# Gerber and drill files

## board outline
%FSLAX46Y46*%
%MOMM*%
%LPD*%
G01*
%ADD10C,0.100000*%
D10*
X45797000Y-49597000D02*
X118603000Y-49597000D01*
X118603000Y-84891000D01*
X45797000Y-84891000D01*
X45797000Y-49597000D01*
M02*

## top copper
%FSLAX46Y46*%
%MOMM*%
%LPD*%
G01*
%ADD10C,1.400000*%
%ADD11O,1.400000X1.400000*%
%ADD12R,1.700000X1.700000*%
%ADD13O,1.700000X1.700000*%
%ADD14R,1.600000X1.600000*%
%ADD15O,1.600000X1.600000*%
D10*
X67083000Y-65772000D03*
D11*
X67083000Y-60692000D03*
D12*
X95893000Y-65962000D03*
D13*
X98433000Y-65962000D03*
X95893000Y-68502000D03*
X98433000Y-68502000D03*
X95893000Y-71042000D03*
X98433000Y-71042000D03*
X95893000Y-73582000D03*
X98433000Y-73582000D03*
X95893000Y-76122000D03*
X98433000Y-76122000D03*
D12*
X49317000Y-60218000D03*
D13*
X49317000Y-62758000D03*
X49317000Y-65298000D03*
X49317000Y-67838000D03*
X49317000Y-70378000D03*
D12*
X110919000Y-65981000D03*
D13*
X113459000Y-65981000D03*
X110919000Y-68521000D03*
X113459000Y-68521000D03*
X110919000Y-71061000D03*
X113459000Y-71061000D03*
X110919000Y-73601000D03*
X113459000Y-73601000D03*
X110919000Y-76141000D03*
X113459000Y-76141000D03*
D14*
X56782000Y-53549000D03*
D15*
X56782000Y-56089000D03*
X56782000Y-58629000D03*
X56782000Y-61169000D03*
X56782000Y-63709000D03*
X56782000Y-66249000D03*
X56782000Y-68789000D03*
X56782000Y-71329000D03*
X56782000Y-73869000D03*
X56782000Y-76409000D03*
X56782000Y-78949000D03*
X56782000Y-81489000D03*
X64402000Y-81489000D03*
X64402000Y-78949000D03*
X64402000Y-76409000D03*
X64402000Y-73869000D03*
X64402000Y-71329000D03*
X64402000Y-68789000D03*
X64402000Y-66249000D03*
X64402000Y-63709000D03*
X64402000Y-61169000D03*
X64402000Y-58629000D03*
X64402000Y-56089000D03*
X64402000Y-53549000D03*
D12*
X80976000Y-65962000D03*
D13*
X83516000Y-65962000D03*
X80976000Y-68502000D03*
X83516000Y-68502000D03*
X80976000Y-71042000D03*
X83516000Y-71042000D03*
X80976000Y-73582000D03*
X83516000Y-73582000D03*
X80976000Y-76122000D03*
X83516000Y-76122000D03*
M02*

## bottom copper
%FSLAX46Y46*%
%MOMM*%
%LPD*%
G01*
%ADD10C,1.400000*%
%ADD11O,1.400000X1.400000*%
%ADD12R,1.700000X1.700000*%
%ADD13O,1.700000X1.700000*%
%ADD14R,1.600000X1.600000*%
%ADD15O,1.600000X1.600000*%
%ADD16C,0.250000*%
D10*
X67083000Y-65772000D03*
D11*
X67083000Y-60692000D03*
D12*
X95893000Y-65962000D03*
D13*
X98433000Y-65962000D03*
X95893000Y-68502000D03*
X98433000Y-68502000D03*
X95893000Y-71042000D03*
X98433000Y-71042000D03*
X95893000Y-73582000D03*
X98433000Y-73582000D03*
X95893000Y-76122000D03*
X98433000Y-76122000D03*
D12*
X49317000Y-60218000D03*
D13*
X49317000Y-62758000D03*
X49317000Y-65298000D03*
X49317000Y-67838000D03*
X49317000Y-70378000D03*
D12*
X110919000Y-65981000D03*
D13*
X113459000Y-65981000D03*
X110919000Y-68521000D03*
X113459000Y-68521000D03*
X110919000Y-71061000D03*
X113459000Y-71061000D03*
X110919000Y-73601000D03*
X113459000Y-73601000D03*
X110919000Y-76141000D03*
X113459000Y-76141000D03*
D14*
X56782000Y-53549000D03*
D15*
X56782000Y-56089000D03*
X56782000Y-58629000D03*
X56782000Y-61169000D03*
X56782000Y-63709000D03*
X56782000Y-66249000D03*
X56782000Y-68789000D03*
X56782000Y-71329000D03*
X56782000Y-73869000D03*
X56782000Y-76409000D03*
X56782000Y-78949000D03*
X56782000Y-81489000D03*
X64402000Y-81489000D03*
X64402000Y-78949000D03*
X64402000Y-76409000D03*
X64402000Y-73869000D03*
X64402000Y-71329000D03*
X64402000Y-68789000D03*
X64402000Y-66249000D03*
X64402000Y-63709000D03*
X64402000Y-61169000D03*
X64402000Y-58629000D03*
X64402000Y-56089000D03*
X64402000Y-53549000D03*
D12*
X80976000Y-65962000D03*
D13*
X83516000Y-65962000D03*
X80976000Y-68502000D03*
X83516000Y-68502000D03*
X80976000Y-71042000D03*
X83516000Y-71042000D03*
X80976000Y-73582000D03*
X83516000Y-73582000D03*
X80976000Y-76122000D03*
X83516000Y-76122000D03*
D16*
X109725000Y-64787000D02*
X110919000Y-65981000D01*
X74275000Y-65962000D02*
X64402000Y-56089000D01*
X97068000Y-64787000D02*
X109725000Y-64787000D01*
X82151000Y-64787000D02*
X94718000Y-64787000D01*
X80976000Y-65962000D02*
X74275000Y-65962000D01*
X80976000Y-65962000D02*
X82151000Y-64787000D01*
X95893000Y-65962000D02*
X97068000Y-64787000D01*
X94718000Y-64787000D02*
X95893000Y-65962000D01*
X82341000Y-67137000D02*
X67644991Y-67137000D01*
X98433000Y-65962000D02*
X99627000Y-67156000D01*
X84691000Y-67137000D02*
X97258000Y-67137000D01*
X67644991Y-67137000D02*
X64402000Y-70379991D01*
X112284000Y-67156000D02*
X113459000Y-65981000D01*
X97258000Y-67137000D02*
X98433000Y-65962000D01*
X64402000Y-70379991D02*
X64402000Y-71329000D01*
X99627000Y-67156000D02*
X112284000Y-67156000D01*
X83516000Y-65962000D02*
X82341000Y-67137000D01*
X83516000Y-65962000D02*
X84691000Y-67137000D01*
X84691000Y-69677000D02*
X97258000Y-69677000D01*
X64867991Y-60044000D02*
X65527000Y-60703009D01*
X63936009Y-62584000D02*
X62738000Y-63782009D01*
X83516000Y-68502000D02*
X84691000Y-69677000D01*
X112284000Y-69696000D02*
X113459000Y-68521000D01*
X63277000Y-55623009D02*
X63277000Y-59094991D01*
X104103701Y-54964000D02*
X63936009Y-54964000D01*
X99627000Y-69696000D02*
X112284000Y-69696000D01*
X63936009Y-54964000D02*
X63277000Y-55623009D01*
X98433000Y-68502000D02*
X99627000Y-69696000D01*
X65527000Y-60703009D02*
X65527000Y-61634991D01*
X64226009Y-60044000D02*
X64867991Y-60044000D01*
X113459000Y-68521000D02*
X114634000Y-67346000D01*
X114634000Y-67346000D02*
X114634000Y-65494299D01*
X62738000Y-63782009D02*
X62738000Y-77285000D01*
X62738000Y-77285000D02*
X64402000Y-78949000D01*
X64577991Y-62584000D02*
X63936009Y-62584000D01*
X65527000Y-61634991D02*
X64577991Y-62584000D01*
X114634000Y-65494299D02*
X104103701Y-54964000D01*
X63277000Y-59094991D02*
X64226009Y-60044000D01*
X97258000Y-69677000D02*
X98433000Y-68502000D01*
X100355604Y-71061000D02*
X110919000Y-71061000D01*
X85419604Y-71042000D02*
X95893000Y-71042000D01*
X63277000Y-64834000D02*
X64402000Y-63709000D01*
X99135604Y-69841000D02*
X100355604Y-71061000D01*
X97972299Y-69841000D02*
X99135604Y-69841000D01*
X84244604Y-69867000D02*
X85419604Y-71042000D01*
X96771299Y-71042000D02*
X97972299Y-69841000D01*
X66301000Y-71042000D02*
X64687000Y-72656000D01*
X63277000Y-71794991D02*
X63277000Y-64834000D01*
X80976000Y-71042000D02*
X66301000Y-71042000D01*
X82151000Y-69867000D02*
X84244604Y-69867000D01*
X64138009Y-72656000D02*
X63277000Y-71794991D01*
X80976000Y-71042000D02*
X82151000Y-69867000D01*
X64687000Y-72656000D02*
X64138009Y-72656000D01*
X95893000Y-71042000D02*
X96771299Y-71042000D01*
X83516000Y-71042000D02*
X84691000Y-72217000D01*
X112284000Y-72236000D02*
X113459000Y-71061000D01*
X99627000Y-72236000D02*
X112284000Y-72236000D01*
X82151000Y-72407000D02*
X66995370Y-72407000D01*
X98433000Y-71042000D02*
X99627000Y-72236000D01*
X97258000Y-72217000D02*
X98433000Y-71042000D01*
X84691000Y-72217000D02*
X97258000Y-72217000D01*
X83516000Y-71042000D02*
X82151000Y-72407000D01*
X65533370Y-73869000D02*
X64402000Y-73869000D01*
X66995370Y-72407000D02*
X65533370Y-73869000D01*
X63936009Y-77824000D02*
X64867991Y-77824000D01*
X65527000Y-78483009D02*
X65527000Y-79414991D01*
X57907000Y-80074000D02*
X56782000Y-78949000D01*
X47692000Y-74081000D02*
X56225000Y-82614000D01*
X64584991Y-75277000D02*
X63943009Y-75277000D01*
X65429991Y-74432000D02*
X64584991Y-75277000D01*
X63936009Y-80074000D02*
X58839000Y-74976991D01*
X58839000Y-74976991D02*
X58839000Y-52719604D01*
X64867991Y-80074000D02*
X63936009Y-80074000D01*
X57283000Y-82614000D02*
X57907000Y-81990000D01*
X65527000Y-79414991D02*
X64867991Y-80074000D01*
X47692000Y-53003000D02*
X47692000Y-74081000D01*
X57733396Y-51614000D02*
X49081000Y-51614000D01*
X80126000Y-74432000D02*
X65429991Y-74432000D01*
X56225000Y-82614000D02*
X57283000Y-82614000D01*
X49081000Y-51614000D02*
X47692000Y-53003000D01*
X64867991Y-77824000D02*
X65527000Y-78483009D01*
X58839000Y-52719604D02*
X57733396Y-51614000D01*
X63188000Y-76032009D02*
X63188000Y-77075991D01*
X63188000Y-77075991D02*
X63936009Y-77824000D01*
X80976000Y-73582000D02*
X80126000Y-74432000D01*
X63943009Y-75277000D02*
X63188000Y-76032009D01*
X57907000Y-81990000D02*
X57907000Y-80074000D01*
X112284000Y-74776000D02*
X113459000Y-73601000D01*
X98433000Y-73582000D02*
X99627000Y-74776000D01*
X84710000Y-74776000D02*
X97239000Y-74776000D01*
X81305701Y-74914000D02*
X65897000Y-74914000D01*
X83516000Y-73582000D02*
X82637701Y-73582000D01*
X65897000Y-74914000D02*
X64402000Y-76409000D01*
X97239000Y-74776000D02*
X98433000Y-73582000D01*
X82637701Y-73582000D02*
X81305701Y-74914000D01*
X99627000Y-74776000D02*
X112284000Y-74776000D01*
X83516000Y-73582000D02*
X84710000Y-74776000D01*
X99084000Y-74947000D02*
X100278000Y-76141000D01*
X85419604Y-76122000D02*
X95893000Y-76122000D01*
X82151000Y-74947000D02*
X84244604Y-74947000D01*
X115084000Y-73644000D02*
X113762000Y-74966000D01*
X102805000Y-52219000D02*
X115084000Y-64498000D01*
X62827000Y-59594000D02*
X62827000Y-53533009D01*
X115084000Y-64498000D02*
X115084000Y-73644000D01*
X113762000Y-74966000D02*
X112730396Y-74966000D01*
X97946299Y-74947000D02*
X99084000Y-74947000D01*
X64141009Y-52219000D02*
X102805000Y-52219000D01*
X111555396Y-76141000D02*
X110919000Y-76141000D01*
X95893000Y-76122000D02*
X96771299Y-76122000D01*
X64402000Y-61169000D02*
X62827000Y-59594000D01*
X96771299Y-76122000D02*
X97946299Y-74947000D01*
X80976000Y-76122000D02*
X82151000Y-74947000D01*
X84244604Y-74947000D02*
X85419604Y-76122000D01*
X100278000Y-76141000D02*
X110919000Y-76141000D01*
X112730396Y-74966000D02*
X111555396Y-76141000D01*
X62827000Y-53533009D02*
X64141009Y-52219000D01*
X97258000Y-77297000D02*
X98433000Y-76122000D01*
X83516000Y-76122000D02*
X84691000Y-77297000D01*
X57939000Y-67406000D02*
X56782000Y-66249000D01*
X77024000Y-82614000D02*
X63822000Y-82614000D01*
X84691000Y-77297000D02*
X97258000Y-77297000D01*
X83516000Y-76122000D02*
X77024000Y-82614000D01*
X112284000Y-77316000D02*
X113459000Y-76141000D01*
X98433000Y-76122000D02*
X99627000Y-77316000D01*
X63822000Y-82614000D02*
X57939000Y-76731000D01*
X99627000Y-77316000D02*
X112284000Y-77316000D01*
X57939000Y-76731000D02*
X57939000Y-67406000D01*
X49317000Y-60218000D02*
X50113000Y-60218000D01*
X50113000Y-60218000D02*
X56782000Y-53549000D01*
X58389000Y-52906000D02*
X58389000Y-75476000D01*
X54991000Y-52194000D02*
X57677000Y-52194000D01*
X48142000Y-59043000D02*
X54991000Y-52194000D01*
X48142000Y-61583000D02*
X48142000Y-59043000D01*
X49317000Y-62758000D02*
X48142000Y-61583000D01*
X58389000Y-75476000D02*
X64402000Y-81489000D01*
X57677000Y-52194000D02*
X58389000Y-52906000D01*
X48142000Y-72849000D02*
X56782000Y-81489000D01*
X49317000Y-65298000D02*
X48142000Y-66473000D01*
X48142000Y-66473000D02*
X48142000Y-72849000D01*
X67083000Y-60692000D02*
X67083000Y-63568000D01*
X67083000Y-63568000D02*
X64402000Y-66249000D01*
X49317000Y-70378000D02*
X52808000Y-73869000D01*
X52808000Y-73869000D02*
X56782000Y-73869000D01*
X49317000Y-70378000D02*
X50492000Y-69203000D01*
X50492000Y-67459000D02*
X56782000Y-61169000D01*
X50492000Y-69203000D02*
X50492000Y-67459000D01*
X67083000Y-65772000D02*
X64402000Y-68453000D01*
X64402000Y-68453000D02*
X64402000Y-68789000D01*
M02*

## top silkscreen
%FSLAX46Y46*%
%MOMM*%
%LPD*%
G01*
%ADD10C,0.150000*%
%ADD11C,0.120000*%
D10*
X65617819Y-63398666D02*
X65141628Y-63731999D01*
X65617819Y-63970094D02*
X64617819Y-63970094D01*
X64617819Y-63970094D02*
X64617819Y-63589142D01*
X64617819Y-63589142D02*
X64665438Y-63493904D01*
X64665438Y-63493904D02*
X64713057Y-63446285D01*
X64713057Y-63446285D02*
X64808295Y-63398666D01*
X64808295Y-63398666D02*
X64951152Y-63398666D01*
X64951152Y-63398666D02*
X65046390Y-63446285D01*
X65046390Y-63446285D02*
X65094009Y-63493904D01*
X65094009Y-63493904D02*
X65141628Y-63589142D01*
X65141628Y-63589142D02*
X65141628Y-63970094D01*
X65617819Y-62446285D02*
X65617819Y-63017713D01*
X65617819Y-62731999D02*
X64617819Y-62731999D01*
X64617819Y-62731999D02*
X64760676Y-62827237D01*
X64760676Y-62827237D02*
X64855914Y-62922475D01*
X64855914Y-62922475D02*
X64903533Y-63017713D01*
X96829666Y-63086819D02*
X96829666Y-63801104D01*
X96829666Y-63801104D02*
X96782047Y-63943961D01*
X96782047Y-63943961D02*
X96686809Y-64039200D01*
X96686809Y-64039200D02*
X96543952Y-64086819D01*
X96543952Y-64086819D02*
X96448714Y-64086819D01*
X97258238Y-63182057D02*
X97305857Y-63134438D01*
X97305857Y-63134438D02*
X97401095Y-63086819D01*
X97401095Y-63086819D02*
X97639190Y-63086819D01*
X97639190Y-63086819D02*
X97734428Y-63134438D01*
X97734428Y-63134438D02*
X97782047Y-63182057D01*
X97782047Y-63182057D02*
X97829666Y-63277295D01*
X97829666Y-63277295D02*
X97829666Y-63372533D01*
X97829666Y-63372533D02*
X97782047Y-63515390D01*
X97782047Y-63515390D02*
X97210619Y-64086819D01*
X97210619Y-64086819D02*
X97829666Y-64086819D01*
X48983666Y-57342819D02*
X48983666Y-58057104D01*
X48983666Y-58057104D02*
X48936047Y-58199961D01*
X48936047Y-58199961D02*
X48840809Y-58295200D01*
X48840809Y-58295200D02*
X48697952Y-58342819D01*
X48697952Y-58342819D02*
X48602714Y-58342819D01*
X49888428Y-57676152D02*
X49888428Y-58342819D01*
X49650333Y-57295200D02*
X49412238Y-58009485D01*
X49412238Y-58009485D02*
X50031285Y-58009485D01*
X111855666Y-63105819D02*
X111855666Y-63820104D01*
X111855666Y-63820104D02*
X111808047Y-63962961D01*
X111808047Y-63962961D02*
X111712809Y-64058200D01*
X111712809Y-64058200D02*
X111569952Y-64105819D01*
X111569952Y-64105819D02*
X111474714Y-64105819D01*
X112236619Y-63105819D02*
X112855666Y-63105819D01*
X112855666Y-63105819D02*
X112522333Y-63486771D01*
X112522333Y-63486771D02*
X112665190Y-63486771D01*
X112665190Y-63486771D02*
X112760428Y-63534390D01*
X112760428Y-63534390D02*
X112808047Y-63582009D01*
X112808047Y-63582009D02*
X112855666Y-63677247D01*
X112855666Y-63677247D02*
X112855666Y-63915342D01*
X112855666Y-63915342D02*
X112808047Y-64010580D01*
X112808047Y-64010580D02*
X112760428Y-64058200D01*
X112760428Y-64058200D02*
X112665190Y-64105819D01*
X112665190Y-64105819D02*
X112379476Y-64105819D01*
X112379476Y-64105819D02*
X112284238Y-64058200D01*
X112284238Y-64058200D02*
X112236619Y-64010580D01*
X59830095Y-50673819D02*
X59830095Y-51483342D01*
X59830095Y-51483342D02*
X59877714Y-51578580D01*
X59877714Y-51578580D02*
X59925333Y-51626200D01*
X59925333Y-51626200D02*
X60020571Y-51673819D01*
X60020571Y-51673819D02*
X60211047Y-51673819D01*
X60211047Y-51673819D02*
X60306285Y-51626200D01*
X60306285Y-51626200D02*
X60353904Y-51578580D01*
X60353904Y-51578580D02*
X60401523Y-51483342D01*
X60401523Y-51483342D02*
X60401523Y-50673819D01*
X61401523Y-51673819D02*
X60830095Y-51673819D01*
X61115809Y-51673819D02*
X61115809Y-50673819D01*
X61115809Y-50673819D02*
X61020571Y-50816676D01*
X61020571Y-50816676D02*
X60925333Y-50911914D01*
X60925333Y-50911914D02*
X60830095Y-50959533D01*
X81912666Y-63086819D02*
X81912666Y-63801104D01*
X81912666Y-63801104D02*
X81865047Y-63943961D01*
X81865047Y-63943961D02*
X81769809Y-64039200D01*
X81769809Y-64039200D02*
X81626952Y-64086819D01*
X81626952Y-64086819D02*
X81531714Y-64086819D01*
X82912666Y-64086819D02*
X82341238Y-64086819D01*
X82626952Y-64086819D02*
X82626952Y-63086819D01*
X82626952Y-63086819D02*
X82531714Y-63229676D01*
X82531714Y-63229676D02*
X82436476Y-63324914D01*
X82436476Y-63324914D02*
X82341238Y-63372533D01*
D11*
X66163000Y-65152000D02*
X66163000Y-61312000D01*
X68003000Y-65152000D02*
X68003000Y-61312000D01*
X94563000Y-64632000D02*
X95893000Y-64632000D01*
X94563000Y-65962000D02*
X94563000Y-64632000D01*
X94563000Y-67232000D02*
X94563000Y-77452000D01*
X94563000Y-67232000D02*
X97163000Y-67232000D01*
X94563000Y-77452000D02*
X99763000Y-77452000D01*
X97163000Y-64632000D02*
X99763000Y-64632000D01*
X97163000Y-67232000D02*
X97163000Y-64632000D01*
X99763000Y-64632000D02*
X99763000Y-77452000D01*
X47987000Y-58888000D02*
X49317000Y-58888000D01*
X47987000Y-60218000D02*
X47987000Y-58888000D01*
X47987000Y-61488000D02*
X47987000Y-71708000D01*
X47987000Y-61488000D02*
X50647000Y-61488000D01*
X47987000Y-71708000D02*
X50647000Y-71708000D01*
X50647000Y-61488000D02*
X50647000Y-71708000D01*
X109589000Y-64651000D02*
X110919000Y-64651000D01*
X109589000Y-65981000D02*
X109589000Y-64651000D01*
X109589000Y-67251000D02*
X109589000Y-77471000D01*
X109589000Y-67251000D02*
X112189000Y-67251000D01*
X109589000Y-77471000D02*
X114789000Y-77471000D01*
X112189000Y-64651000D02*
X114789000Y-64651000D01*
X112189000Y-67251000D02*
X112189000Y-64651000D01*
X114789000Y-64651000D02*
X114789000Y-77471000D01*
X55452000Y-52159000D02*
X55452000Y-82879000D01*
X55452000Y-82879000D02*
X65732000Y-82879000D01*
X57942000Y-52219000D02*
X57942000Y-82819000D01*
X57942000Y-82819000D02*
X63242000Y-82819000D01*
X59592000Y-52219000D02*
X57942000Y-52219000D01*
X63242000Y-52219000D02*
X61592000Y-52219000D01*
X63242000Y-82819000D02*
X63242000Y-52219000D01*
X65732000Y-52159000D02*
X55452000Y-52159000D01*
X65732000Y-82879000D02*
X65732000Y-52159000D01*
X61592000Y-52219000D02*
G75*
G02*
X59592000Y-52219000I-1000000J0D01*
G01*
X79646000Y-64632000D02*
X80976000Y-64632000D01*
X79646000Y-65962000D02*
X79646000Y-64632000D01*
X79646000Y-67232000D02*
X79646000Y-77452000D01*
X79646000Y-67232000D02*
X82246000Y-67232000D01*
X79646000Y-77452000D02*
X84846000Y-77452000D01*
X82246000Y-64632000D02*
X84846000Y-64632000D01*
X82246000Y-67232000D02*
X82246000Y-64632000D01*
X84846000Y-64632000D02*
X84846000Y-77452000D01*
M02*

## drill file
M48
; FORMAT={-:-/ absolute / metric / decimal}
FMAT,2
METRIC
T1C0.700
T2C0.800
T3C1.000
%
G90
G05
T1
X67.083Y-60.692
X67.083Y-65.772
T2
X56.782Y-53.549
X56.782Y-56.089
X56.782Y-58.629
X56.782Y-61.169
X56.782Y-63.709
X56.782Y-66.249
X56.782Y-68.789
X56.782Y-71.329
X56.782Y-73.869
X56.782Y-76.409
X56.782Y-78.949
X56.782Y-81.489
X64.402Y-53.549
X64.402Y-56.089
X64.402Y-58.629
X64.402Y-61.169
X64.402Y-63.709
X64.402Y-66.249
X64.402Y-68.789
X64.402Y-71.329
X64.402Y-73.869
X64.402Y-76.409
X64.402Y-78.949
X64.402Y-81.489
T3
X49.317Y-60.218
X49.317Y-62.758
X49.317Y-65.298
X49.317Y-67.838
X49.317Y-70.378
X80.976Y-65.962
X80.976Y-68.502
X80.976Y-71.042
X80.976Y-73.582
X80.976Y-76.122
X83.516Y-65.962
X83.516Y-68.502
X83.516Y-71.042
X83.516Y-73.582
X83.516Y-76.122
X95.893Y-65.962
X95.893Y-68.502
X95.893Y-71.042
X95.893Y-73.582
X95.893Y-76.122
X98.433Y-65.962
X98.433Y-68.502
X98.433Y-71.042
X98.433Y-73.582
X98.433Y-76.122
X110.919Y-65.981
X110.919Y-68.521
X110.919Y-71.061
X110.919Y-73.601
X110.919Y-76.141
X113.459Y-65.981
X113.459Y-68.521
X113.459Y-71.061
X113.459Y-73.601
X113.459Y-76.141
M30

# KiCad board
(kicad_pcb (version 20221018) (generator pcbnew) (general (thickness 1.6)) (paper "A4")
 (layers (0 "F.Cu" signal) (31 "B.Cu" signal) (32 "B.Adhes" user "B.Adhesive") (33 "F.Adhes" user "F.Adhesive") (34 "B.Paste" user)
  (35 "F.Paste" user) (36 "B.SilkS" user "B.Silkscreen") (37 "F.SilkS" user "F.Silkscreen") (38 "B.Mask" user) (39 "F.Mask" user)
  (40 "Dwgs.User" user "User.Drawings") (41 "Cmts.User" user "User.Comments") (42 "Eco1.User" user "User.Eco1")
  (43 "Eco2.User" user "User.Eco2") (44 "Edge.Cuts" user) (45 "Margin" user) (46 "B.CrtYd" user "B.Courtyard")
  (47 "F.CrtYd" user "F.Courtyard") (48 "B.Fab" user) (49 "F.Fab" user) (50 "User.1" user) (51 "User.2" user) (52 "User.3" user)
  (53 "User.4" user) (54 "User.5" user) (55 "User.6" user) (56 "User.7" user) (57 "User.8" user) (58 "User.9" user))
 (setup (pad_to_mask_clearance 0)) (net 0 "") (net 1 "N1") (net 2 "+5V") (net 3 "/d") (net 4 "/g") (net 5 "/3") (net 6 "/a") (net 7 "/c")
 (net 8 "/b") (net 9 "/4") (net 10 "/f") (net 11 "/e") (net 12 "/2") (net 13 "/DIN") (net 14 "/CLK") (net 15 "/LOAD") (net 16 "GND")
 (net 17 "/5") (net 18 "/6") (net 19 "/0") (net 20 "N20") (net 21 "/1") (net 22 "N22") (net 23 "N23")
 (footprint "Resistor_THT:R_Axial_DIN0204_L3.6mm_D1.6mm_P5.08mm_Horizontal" (layer "F.Cu") (at 67.083 65.772 90)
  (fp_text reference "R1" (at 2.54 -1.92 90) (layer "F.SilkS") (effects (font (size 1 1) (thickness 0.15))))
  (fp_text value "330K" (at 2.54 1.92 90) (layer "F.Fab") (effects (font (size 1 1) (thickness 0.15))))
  (fp_line (start 0.62 -0.92) (end 4.46 -0.92) (stroke (width 0.12) (type solid)) (layer "F.SilkS"))
  (fp_line (start 0.62 0.92) (end 4.46 0.92) (stroke (width 0.12) (type solid)) (layer "F.SilkS"))
  (pad "1" thru_hole circle (at 0 0 90) (size 1.4 1.4) (drill 0.7) (layers "*.Cu" "*.Mask") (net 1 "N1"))
  (pad "2" thru_hole oval (at 5.08 0 90) (size 1.4 1.4) (drill 0.7) (layers "*.Cu" "*.Mask") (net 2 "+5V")))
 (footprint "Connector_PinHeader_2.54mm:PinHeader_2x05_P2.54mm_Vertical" (layer "F.Cu") (at 95.893 65.962)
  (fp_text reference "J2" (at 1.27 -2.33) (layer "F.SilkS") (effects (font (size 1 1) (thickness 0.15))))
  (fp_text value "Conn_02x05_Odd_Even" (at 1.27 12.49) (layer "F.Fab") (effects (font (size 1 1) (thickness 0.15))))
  (fp_line (start -1.33 -1.33) (end 0 -1.33) (stroke (width 0.12) (type solid)) (layer "F.SilkS"))
  (fp_line (start -1.33 0) (end -1.33 -1.33) (stroke (width 0.12) (type solid)) (layer "F.SilkS"))
  (fp_line (start -1.33 1.27) (end -1.33 11.49) (stroke (width 0.12) (type solid)) (layer "F.SilkS"))
  (fp_line (start -1.33 1.27) (end 1.27 1.27) (stroke (width 0.12) (type solid)) (layer "F.SilkS"))
  (fp_line (start -1.33 11.49) (end 3.87 11.49) (stroke (width 0.12) (type solid)) (layer "F.SilkS"))
  (fp_line (start 1.27 -1.33) (end 3.87 -1.33) (stroke (width 0.12) (type solid)) (layer "F.SilkS"))
  (fp_line (start 1.27 1.27) (end 1.27 -1.33) (stroke (width 0.12) (type solid)) (layer "F.SilkS"))
  (fp_line (start 3.87 -1.33) (end 3.87 11.49) (stroke (width 0.12) (type solid)) (layer "F.SilkS"))
  (pad "1" thru_hole rect (at 0 0) (size 1.7 1.7) (drill 1) (layers "*.Cu" "*.Mask") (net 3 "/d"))
  (pad "2" thru_hole oval (at 2.54 0) (size 1.7 1.7) (drill 1) (layers "*.Cu" "*.Mask") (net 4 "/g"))
  (pad "3" thru_hole oval (at 0 2.54) (size 1.7 1.7) (drill 1) (layers "*.Cu" "*.Mask") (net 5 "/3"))
  (pad "4" thru_hole oval (at 2.54 2.54) (size 1.7 1.7) (drill 1) (layers "*.Cu" "*.Mask") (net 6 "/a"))
  (pad "5" thru_hole oval (at 0 5.08) (size 1.7 1.7) (drill 1) (layers "*.Cu" "*.Mask") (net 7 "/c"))
  (pad "6" thru_hole oval (at 2.54 5.08) (size 1.7 1.7) (drill 1) (layers "*.Cu" "*.Mask") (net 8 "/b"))
  (pad "7" thru_hole oval (at 0 7.62) (size 1.7 1.7) (drill 1) (layers "*.Cu" "*.Mask") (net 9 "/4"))
  (pad "8" thru_hole oval (at 2.54 7.62) (size 1.7 1.7) (drill 1) (layers "*.Cu" "*.Mask") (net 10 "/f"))
  (pad "9" thru_hole oval (at 0 10.16) (size 1.7 1.7) (drill 1) (layers "*.Cu" "*.Mask") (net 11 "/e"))
  (pad "10" thru_hole oval (at 2.54 10.16) (size 1.7 1.7) (drill 1) (layers "*.Cu" "*.Mask") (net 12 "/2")))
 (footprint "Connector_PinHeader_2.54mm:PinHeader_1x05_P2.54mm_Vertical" (layer "F.Cu") (at 49.317 60.218)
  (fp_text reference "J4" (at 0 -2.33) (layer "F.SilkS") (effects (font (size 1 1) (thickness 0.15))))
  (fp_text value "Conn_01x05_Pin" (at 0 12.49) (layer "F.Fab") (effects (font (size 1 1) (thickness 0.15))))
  (fp_line (start -1.33 -1.33) (end 0 -1.33) (stroke (width 0.12) (type solid)) (layer "F.SilkS"))
  (fp_line (start -1.33 0) (end -1.33 -1.33) (stroke (width 0.12) (type solid)) (layer "F.SilkS"))
  (fp_line (start -1.33 1.27) (end -1.33 11.49) (stroke (width 0.12) (type solid)) (layer "F.SilkS"))
  (fp_line (start -1.33 1.27) (end 1.33 1.27) (stroke (width 0.12) (type solid)) (layer "F.SilkS"))
  (fp_line (start -1.33 11.49) (end 1.33 11.49) (stroke (width 0.12) (type solid)) (layer "F.SilkS"))
  (fp_line (start 1.33 1.27) (end 1.33 11.49) (stroke (width 0.12) (type solid)) (layer "F.SilkS"))
  (pad "1" thru_hole rect (at 0 0) (size 1.7 1.7) (drill 1) (layers "*.Cu" "*.Mask") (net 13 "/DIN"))
  (pad "2" thru_hole oval (at 0 2.54) (size 1.7 1.7) (drill 1) (layers "*.Cu" "*.Mask") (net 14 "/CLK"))
  (pad "3" thru_hole oval (at 0 5.08) (size 1.7 1.7) (drill 1) (layers "*.Cu" "*.Mask") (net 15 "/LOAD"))
  (pad "4" thru_hole oval (at 0 7.62) (size 1.7 1.7) (drill 1) (layers "*.Cu" "*.Mask") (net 2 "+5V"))
  (pad "5" thru_hole oval (at 0 10.16) (size 1.7 1.7) (drill 1) (layers "*.Cu" "*.Mask") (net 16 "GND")))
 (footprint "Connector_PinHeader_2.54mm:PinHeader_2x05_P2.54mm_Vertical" (layer "F.Cu") (at 110.919 65.981)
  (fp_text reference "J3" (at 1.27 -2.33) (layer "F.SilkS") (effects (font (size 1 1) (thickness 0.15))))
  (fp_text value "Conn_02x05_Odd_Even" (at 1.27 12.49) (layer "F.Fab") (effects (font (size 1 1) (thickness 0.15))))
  (fp_line (start -1.33 -1.33) (end 0 -1.33) (stroke (width 0.12) (type solid)) (layer "F.SilkS"))
  (fp_line (start -1.33 0) (end -1.33 -1.33) (stroke (width 0.12) (type solid)) (layer "F.SilkS"))
  (fp_line (start -1.33 1.27) (end -1.33 11.49) (stroke (width 0.12) (type solid)) (layer "F.SilkS"))
  (fp_line (start -1.33 1.27) (end 1.27 1.27) (stroke (width 0.12) (type solid)) (layer "F.SilkS"))
  (fp_line (start -1.33 11.49) (end 3.87 11.49) (stroke (width 0.12) (type solid)) (layer "F.SilkS"))
  (fp_line (start 1.27 -1.33) (end 3.87 -1.33) (stroke (width 0.12) (type solid)) (layer "F.SilkS"))
  (fp_line (start 1.27 1.27) (end 1.27 -1.33) (stroke (width 0.12) (type solid)) (layer "F.SilkS"))
  (fp_line (start 3.87 -1.33) (end 3.87 11.49) (stroke (width 0.12) (type solid)) (layer "F.SilkS"))
  (pad "1" thru_hole rect (at 0 0) (size 1.7 1.7) (drill 1) (layers "*.Cu" "*.Mask") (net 3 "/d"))
  (pad "2" thru_hole oval (at 2.54 0) (size 1.7 1.7) (drill 1) (layers "*.Cu" "*.Mask") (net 4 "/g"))
  (pad "3" thru_hole oval (at 0 2.54) (size 1.7 1.7) (drill 1) (layers "*.Cu" "*.Mask") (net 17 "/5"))
  (pad "4" thru_hole oval (at 2.54 2.54) (size 1.7 1.7) (drill 1) (layers "*.Cu" "*.Mask") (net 6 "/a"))
  (pad "5" thru_hole oval (at 0 5.08) (size 1.7 1.7) (drill 1) (layers "*.Cu" "*.Mask") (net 7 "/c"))
  (pad "6" thru_hole oval (at 2.54 5.08) (size 1.7 1.7) (drill 1) (layers "*.Cu" "*.Mask") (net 8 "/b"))
  (pad "7" thru_hole oval (at 0 7.62) (size 1.7 1.7) (drill 1) (layers "*.Cu" "*.Mask") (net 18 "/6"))
  (pad "8" thru_hole oval (at 2.54 7.62) (size 1.7 1.7) (drill 1) (layers "*.Cu" "*.Mask") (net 10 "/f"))
  (pad "9" thru_hole oval (at 0 10.16) (size 1.7 1.7) (drill 1) (layers "*.Cu" "*.Mask") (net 11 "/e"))
  (pad "10" thru_hole oval (at 2.54 10.16) (size 1.7 1.7) (drill 1) (layers "*.Cu" "*.Mask") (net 12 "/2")))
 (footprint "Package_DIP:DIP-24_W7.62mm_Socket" (layer "F.Cu") (at 56.782 53.549)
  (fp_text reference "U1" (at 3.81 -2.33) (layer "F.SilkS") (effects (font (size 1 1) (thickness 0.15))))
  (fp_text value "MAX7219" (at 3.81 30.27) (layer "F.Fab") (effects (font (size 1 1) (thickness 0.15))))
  (fp_line (start -1.33 -1.39) (end -1.33 29.33) (stroke (width 0.12) (type solid)) (layer "F.SilkS"))
  (fp_line (start -1.33 29.33) (end 8.95 29.33) (stroke (width 0.12) (type solid)) (layer "F.SilkS"))
  (fp_line (start 1.16 -1.33) (end 1.16 29.27) (stroke (width 0.12) (type solid)) (layer "F.SilkS"))
  (fp_line (start 1.16 29.27) (end 6.46 29.27) (stroke (width 0.12) (type solid)) (layer "F.SilkS"))
  (fp_line (start 2.81 -1.33) (end 1.16 -1.33) (stroke (width 0.12) (type solid)) (layer "F.SilkS"))
  (fp_line (start 6.46 -1.33) (end 4.81 -1.33) (stroke (width 0.12) (type solid)) (layer "F.SilkS"))
  (fp_line (start 6.46 29.27) (end 6.46 -1.33) (stroke (width 0.12) (type solid)) (layer "F.SilkS"))
  (fp_line (start 8.95 -1.39) (end -1.33 -1.39) (stroke (width 0.12) (type solid)) (layer "F.SilkS"))
  (fp_line (start 8.95 29.33) (end 8.95 -1.39) (stroke (width 0.12) (type solid)) (layer "F.SilkS"))
  (fp_arc (start 4.81 -1.33) (mid 3.81 -0.33) (end 2.81 -1.33) (stroke (width 0.12) (type solid)) (layer "F.SilkS"))
  (pad "1" thru_hole rect (at 0 0) (size 1.6 1.6) (drill 0.8) (layers "*.Cu" "*.Mask") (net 13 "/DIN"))
  (pad "2" thru_hole oval (at 0 2.54) (size 1.6 1.6) (drill 0.8) (layers "*.Cu" "*.Mask") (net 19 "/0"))
  (pad "3" thru_hole oval (at 0 5.08) (size 1.6 1.6) (drill 0.8) (layers "*.Cu" "*.Mask") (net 9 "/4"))
  (pad "4" thru_hole oval (at 0 7.62) (size 1.6 1.6) (drill 0.8) (layers "*.Cu" "*.Mask") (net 16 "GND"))
  (pad "5" thru_hole oval (at 0 10.16) (size 1.6 1.6) (drill 0.8) (layers "*.Cu" "*.Mask") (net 18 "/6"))
  (pad "6" thru_hole oval (at 0 12.7) (size 1.6 1.6) (drill 0.8) (layers "*.Cu" "*.Mask") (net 12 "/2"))
  (pad "7" thru_hole oval (at 0 15.24) (size 1.6 1.6) (drill 0.8) (layers "*.Cu" "*.Mask") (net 5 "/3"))
  (pad "8" thru_hole oval (at 0 17.78) (size 1.6 1.6) (drill 0.8) (layers "*.Cu" "*.Mask") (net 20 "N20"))
  (pad "9" thru_hole oval (at 0 20.32) (size 1.6 1.6) (drill 0.8) (layers "*.Cu" "*.Mask") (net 16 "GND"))
  (pad "10" thru_hole oval (at 0 22.86) (size 1.6 1.6) (drill 0.8) (layers "*.Cu" "*.Mask") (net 17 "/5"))
  (pad "11" thru_hole oval (at 0 25.4) (size 1.6 1.6) (drill 0.8) (layers "*.Cu" "*.Mask") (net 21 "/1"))
  (pad "12" thru_hole oval (at 0 27.94) (size 1.6 1.6) (drill 0.8) (layers "*.Cu" "*.Mask") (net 15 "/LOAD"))
  (pad "13" thru_hole oval (at 7.62 27.94) (size 1.6 1.6) (drill 0.8) (layers "*.Cu" "*.Mask") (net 14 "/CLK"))
  (pad "14" thru_hole oval (at 7.62 25.4) (size 1.6 1.6) (drill 0.8) (layers "*.Cu" "*.Mask") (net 6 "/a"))
  (pad "15" thru_hole oval (at 7.62 22.86) (size 1.6 1.6) (drill 0.8) (layers "*.Cu" "*.Mask") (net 10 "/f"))
  (pad "16" thru_hole oval (at 7.62 20.32) (size 1.6 1.6) (drill 0.8) (layers "*.Cu" "*.Mask") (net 8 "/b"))
  (pad "17" thru_hole oval (at 7.62 17.78) (size 1.6 1.6) (drill 0.8) (layers "*.Cu" "*.Mask") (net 4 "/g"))
  (pad "18" thru_hole oval (at 7.62 15.24) (size 1.6 1.6) (drill 0.8) (layers "*.Cu" "*.Mask") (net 1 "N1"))
  (pad "19" thru_hole oval (at 7.62 12.7) (size 1.6 1.6) (drill 0.8) (layers "*.Cu" "*.Mask") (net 2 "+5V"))
  (pad "20" thru_hole oval (at 7.62 10.16) (size 1.6 1.6) (drill 0.8) (layers "*.Cu" "*.Mask") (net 7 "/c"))
  (pad "21" thru_hole oval (at 7.62 7.62) (size 1.6 1.6) (drill 0.8) (layers "*.Cu" "*.Mask") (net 11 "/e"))
  (pad "22" thru_hole oval (at 7.62 5.08) (size 1.6 1.6) (drill 0.8) (layers "*.Cu" "*.Mask") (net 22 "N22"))
  (pad "23" thru_hole oval (at 7.62 2.54) (size 1.6 1.6) (drill 0.8) (layers "*.Cu" "*.Mask") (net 3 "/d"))
  (pad "24" thru_hole oval (at 7.62 0) (size 1.6 1.6) (drill 0.8) (layers "*.Cu" "*.Mask") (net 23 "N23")))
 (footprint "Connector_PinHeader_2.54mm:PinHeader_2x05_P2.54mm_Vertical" (layer "F.Cu") (at 80.976 65.962)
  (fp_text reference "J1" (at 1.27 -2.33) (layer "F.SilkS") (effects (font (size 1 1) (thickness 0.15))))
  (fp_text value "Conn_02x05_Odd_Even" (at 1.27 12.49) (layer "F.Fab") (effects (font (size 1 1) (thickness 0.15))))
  (fp_line (start -1.33 -1.33) (end 0 -1.33) (stroke (width 0.12) (type solid)) (layer "F.SilkS"))
  (fp_line (start -1.33 0) (end -1.33 -1.33) (stroke (width 0.12) (type solid)) (layer "F.SilkS"))
  (fp_line (start -1.33 1.27) (end -1.33 11.49) (stroke (width 0.12) (type solid)) (layer "F.SilkS"))
  (fp_line (start -1.33 1.27) (end 1.27 1.27) (stroke (width 0.12) (type solid)) (layer "F.SilkS"))
  (fp_line (start -1.33 11.49) (end 3.87 11.49) (stroke (width 0.12) (type solid)) (layer "F.SilkS"))
  (fp_line (start 1.27 -1.33) (end 3.87 -1.33) (stroke (width 0.12) (type solid)) (layer "F.SilkS"))
  (fp_line (start 1.27 1.27) (end 1.27 -1.33) (stroke (width 0.12) (type solid)) (layer "F.SilkS"))
  (fp_line (start 3.87 -1.33) (end 3.87 11.49) (stroke (width 0.12) (type solid)) (layer "F.SilkS"))
  (pad "1" thru_hole rect (at 0 0) (size 1.7 1.7) (drill 1) (layers "*.Cu" "*.Mask") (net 3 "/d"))
  (pad "2" thru_hole oval (at 2.54 0) (size 1.7 1.7) (drill 1) (layers "*.Cu" "*.Mask") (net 4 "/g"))
  (pad "3" thru_hole oval (at 0 2.54) (size 1.7 1.7) (drill 1) (layers "*.Cu" "*.Mask") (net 19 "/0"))
  (pad "4" thru_hole oval (at 2.54 2.54) (size 1.7 1.7) (drill 1) (layers "*.Cu" "*.Mask") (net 6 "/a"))
  (pad "5" thru_hole oval (at 0 5.08) (size 1.7 1.7) (drill 1) (layers "*.Cu" "*.Mask") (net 7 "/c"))
  (pad "6" thru_hole oval (at 2.54 5.08) (size 1.7 1.7) (drill 1) (layers "*.Cu" "*.Mask") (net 8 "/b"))
  (pad "7" thru_hole oval (at 0 7.62) (size 1.7 1.7) (drill 1) (layers "*.Cu" "*.Mask") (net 21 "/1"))
  (pad "8" thru_hole oval (at 2.54 7.62) (size 1.7 1.7) (drill 1) (layers "*.Cu" "*.Mask") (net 10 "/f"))
  (pad "9" thru_hole oval (at 0 10.16) (size 1.7 1.7) (drill 1) (layers "*.Cu" "*.Mask") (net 11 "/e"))
  (pad "10" thru_hole oval (at 2.54 10.16) (size 1.7 1.7) (drill 1) (layers "*.Cu" "*.Mask") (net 12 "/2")))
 (gr_rect (start 45.797 49.597) (end 118.603 84.891) (stroke (width 0.1) (type default)) (fill none) (layer "Edge.Cuts"))
 (segment (start 109.725 64.787) (end 110.919 65.981) (width 0.25) (layer "B.Cu") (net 3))
 (segment (start 74.275 65.962) (end 64.402 56.089) (width 0.25) (layer "B.Cu") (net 3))
 (segment (start 97.068 64.787) (end 109.725 64.787) (width 0.25) (layer "B.Cu") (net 3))
 (segment (start 82.151 64.787) (end 94.718 64.787) (width 0.25) (layer "B.Cu") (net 3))
 (segment (start 80.976 65.962) (end 74.275 65.962) (width 0.25) (layer "B.Cu") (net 3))
 (segment (start 80.976 65.962) (end 82.151 64.787) (width 0.25) (layer "B.Cu") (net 3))
 (segment (start 95.893 65.962) (end 97.068 64.787) (width 0.25) (layer "B.Cu") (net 3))
 (segment (start 94.718 64.787) (end 95.893 65.962) (width 0.25) (layer "B.Cu") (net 3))
 (segment (start 82.341 67.137) (end 67.644991 67.137) (width 0.25) (layer "B.Cu") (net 4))
 (segment (start 98.433 65.962) (end 99.627 67.156) (width 0.25) (layer "B.Cu") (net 4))
 (segment (start 84.691 67.137) (end 97.258 67.137) (width 0.25) (layer "B.Cu") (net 4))
 (segment (start 67.644991 67.137) (end 64.402 70.379991) (width 0.25) (layer "B.Cu") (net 4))
 (segment (start 112.284 67.156) (end 113.459 65.981) (width 0.25) (layer "B.Cu") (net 4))
 (segment (start 97.258 67.137) (end 98.433 65.962) (width 0.25) (layer "B.Cu") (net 4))
 (segment (start 64.402 70.379991) (end 64.402 71.329) (width 0.25) (layer "B.Cu") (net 4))
 (segment (start 99.627 67.156) (end 112.284 67.156) (width 0.25) (layer "B.Cu") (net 4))
 (segment (start 83.516 65.962) (end 82.341 67.137) (width 0.25) (layer "B.Cu") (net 4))
 (segment (start 83.516 65.962) (end 84.691 67.137) (width 0.25) (layer "B.Cu") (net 4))
 (segment (start 84.691 69.677) (end 97.258 69.677) (width 0.25) (layer "B.Cu") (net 6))
 (segment (start 64.867991 60.044) (end 65.527 60.703009) (width 0.25) (layer "B.Cu") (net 6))
 (segment (start 63.936009 62.584) (end 62.738 63.782009) (width 0.25) (layer "B.Cu") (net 6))
 (segment (start 83.516 68.502) (end 84.691 69.677) (width 0.25) (layer "B.Cu") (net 6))
 (segment (start 112.284 69.696) (end 113.459 68.521) (width 0.25) (layer "B.Cu") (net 6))
 (segment (start 63.277 55.623009) (end 63.277 59.094991) (width 0.25) (layer "B.Cu") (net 6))
 (segment (start 104.103701 54.964) (end 63.936009 54.964) (width 0.25) (layer "B.Cu") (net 6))
 (segment (start 99.627 69.696) (end 112.284 69.696) (width 0.25) (layer "B.Cu") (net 6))
 (segment (start 63.936009 54.964) (end 63.277 55.623009) (width 0.25) (layer "B.Cu") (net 6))
 (segment (start 98.433 68.502) (end 99.627 69.696) (width 0.25) (layer "B.Cu") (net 6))
 (segment (start 65.527 60.703009) (end 65.527 61.634991) (width 0.25) (layer "B.Cu") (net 6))
 (segment (start 64.226009 60.044) (end 64.867991 60.044) (width 0.25) (layer "B.Cu") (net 6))
 (segment (start 113.459 68.521) (end 114.634 67.346) (width 0.25) (layer "B.Cu") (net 6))
 (segment (start 114.634 67.346) (end 114.634 65.494299) (width 0.25) (layer "B.Cu") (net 6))
 (segment (start 62.738 63.782009) (end 62.738 77.285) (width 0.25) (layer "B.Cu") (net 6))
 (segment (start 62.738 77.285) (end 64.402 78.949) (width 0.25) (layer "B.Cu") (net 6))
 (segment (start 64.577991 62.584) (end 63.936009 62.584) (width 0.25) (layer "B.Cu") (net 6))
 (segment (start 65.527 61.634991) (end 64.577991 62.584) (width 0.25) (layer "B.Cu") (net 6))
 (segment (start 114.634 65.494299) (end 104.103701 54.964) (width 0.25) (layer "B.Cu") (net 6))
 (segment (start 63.277 59.094991) (end 64.226009 60.044) (width 0.25) (layer "B.Cu") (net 6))
 (segment (start 97.258 69.677) (end 98.433 68.502) (width 0.25) (layer "B.Cu") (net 6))
 (segment (start 100.355604 71.061) (end 110.919 71.061) (width 0.25) (layer "B.Cu") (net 7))
 (segment (start 85.419604 71.042) (end 95.893 71.042) (width 0.25) (layer "B.Cu") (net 7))
 (segment (start 63.277 64.834) (end 64.402 63.709) (width 0.25) (layer "B.Cu") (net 7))
 (segment (start 99.135604 69.841) (end 100.355604 71.061) (width 0.25) (layer "B.Cu") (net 7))
 (segment (start 97.972299 69.841) (end 99.135604 69.841) (width 0.25) (layer "B.Cu") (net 7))
 (segment (start 84.244604 69.867) (end 85.419604 71.042) (width 0.25) (layer "B.Cu") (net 7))
 (segment (start 96.771299 71.042) (end 97.972299 69.841) (width 0.25) (layer "B.Cu") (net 7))
 (segment (start 66.301 71.042) (end 64.687 72.656) (width 0.25) (layer "B.Cu") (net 7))
 (segment (start 63.277 71.794991) (end 63.277 64.834) (width 0.25) (layer "B.Cu") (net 7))
 (segment (start 80.976 71.042) (end 66.301 71.042) (width 0.25) (layer "B.Cu") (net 7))
 (segment (start 82.151 69.867) (end 84.244604 69.867) (width 0.25) (layer "B.Cu") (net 7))
 (segment (start 64.138009 72.656) (end 63.277 71.794991) (width 0.25) (layer "B.Cu") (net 7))
 (segment (start 80.976 71.042) (end 82.151 69.867) (width 0.25) (layer "B.Cu") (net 7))
 (segment (start 64.687 72.656) (end 64.138009 72.656) (width 0.25) (layer "B.Cu") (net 7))
 (segment (start 95.893 71.042) (end 96.771299 71.042) (width 0.25) (layer "B.Cu") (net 7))
 (segment (start 83.516 71.042) (end 84.691 72.217) (width 0.25) (layer "B.Cu") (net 8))
 (segment (start 112.284 72.236) (end 113.459 71.061) (width 0.25) (layer "B.Cu") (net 8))
 (segment (start 99.627 72.236) (end 112.284 72.236) (width 0.25) (layer "B.Cu") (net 8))
 (segment (start 82.151 72.407) (end 66.99537 72.407) (width 0.25) (layer "B.Cu") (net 8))
 (segment (start 98.433 71.042) (end 99.627 72.236) (width 0.25) (layer "B.Cu") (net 8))
 (segment (start 97.258 72.217) (end 98.433 71.042) (width 0.25) (layer "B.Cu") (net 8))
 (segment (start 84.691 72.217) (end 97.258 72.217) (width 0.25) (layer "B.Cu") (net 8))
 (segment (start 83.516 71.042) (end 82.151 72.407) (width 0.25) (layer "B.Cu") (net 8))
 (segment (start 65.53337 73.869) (end 64.402 73.869) (width 0.25) (layer "B.Cu") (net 8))
 (segment (start 66.99537 72.407) (end 65.53337 73.869) (width 0.25) (layer "B.Cu") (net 8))
 (segment (start 63.936009 77.824) (end 64.867991 77.824) (width 0.25) (layer "B.Cu") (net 21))
 (segment (start 65.527 78.483009) (end 65.527 79.414991) (width 0.25) (layer "B.Cu") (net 21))
 (segment (start 57.907 80.074) (end 56.782 78.949) (width 0.25) (layer "B.Cu") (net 21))
 (segment (start 47.692 74.081) (end 56.225 82.614) (width 0.25) (layer "B.Cu") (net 21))
 (segment (start 64.584991 75.277) (end 63.943009 75.277) (width 0.25) (layer "B.Cu") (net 21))
 (segment (start 65.429991 74.432) (end 64.584991 75.277) (width 0.25) (layer "B.Cu") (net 21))
 (segment (start 63.936009 80.074) (end 58.839 74.976991) (width 0.25) (layer "B.Cu") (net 21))
 (segment (start 58.839 74.976991) (end 58.839 52.719604) (width 0.25) (layer "B.Cu") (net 21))
 (segment (start 64.867991 80.074) (end 63.936009 80.074) (width 0.25) (layer "B.Cu") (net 21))
 (segment (start 57.283 82.614) (end 57.907 81.99) (width 0.25) (layer "B.Cu") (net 21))
 (segment (start 65.527 79.414991) (end 64.867991 80.074) (width 0.25) (layer "B.Cu") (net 21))
 (segment (start 47.692 53.003) (end 47.692 74.081) (width 0.25) (layer "B.Cu") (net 21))
 (segment (start 57.733396 51.614) (end 49.081 51.614) (width 0.25) (layer "B.Cu") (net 21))
 (segment (start 80.126 74.432) (end 65.429991 74.432) (width 0.25) (layer "B.Cu") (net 21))
 (segment (start 56.225 82.614) (end 57.283 82.614) (width 0.25) (layer "B.Cu") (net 21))
 (segment (start 49.081 51.614) (end 47.692 53.003) (width 0.25) (layer "B.Cu") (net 21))
 (segment (start 64.867991 77.824) (end 65.527 78.483009) (width 0.25) (layer "B.Cu") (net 21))
 (segment (start 58.839 52.719604) (end 57.733396 51.614) (width 0.25) (layer "B.Cu") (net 21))
 (segment (start 63.188 76.032009) (end 63.188 77.075991) (width 0.25) (layer "B.Cu") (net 21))
 (segment (start 63.188 77.075991) (end 63.936009 77.824) (width 0.25) (layer "B.Cu") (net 21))
 (segment (start 80.976 73.582) (end 80.126 74.432) (width 0.25) (layer "B.Cu") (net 21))
 (segment (start 63.943009 75.277) (end 63.188 76.032009) (width 0.25) (layer "B.Cu") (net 21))
 (segment (start 57.907 81.99) (end 57.907 80.074) (width 0.25) (layer "B.Cu") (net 21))
 (segment (start 112.284 74.776) (end 113.459 73.601) (width 0.25) (layer "B.Cu") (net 10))
 (segment (start 98.433 73.582) (end 99.627 74.776) (width 0.25) (layer "B.Cu") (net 10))
 (segment (start 84.71 74.776) (end 97.239 74.776) (width 0.25) (layer "B.Cu") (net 10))
 (segment (start 81.305701 74.914) (end 65.897 74.914) (width 0.25) (layer "B.Cu") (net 10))
 (segment (start 83.516 73.582) (end 82.637701 73.582) (width 0.25) (layer "B.Cu") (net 10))
 (segment (start 65.897 74.914) (end 64.402 76.409) (width 0.25) (layer "B.Cu") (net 10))
 (segment (start 97.239 74.776) (end 98.433 73.582) (width 0.25) (layer "B.Cu") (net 10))
 (segment (start 82.637701 73.582) (end 81.305701 74.914) (width 0.25) (layer "B.Cu") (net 10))
 (segment (start 99.627 74.776) (end 112.284 74.776) (width 0.25) (layer "B.Cu") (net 10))
 (segment (start 83.516 73.582) (end 84.71 74.776) (width 0.25) (layer "B.Cu") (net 10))
 (segment (start 99.084 74.947) (end 100.278 76.141) (width 0.25) (layer "B.Cu") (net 11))
 (segment (start 85.419604 76.122) (end 95.893 76.122) (width 0.25) (layer "B.Cu") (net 11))
 (segment (start 82.151 74.947) (end 84.244604 74.947) (width 0.25) (layer "B.Cu") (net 11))
 (segment (start 115.084 73.644) (end 113.762 74.966) (width 0.25) (layer "B.Cu") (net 11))
 (segment (start 102.805 52.219) (end 115.084 64.498) (width 0.25) (layer "B.Cu") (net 11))
 (segment (start 62.827 59.594) (end 62.827 53.533009) (width 0.25) (layer "B.Cu") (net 11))
 (segment (start 115.084 64.498) (end 115.084 73.644) (width 0.25) (layer "B.Cu") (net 11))
 (segment (start 113.762 74.966) (end 112.730396 74.966) (width 0.25) (layer "B.Cu") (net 11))
 (segment (start 97.946299 74.947) (end 99.084 74.947) (width 0.25) (layer "B.Cu") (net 11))
 (segment (start 64.141009 52.219) (end 102.805 52.219) (width 0.25) (layer "B.Cu") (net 11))
 (segment (start 111.555396 76.141) (end 110.919 76.141) (width 0.25) (layer "B.Cu") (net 11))
 (segment (start 95.893 76.122) (end 96.771299 76.122) (width 0.25) (layer "B.Cu") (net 11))
 (segment (start 64.402 61.169) (end 62.827 59.594) (width 0.25) (layer "B.Cu") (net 11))
 (segment (start 96.771299 76.122) (end 97.946299 74.947) (width 0.25) (layer "B.Cu") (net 11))
 (segment (start 80.976 76.122) (end 82.151 74.947) (width 0.25) (layer "B.Cu") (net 11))
 (segment (start 84.244604 74.947) (end 85.419604 76.122) (width 0.25) (layer "B.Cu") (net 11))
 (segment (start 100.278 76.141) (end 110.919 76.141) (width 0.25) (layer "B.Cu") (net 11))
 (segment (start 112.730396 74.966) (end 111.555396 76.141) (width 0.25) (layer "B.Cu") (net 11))
 (segment (start 62.827 53.533009) (end 64.141009 52.219) (width 0.25) (layer "B.Cu") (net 11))
 (segment (start 97.258 77.297) (end 98.433 76.122) (width 0.25) (layer "B.Cu") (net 12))
 (segment (start 83.516 76.122) (end 84.691 77.297) (width 0.25) (layer "B.Cu") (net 12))
 (segment (start 57.939 67.406) (end 56.782 66.249) (width 0.25) (layer "B.Cu") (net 12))
 (segment (start 77.024 82.614) (end 63.822 82.614) (width 0.25) (layer "B.Cu") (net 12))
 (segment (start 84.691 77.297) (end 97.258 77.297) (width 0.25) (layer "B.Cu") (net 12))
 (segment (start 83.516 76.122) (end 77.024 82.614) (width 0.25) (layer "B.Cu") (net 12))
 (segment (start 112.284 77.316) (end 113.459 76.141) (width 0.25) (layer "B.Cu") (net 12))
 (segment (start 98.433 76.122) (end 99.627 77.316) (width 0.25) (layer "B.Cu") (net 12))
 (segment (start 63.822 82.614) (end 57.939 76.731) (width 0.25) (layer "B.Cu") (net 12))
 (segment (start 99.627 77.316) (end 112.284 77.316) (width 0.25) (layer "B.Cu") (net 12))
 (segment (start 57.939 76.731) (end 57.939 67.406) (width 0.25) (layer "B.Cu") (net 12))
 (segment (start 49.317 60.218) (end 50.113 60.218) (width 0.25) (layer "B.Cu") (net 13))
 (segment (start 50.113 60.218) (end 56.782 53.549) (width 0.25) (layer "B.Cu") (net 13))
 (segment (start 58.389 52.906) (end 58.389 75.476) (width 0.25) (layer "B.Cu") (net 14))
 (segment (start 54.991 52.194) (end 57.677 52.194) (width 0.25) (layer "B.Cu") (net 14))
 (segment (start 48.142 59.043) (end 54.991 52.194) (width 0.25) (layer "B.Cu") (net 14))
 (segment (start 48.142 61.583) (end 48.142 59.043) (width 0.25) (layer "B.Cu") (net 14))
 (segment (start 49.317 62.758) (end 48.142 61.583) (width 0.25) (layer "B.Cu") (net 14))
 (segment (start 58.389 75.476) (end 64.402 81.489) (width 0.25) (layer "B.Cu") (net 14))
 (segment (start 57.677 52.194) (end 58.389 52.906) (width 0.25) (layer "B.Cu") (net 14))
 (segment (start 48.142 72.849) (end 56.782 81.489) (width 0.25) (layer "B.Cu") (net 15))
 (segment (start 49.317 65.298) (end 48.142 66.473) (width 0.25) (layer "B.Cu") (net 15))
 (segment (start 48.142 66.473) (end 48.142 72.849) (width 0.25) (layer "B.Cu") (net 15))
 (segment (start 67.083 60.692) (end 67.083 63.568) (width 0.25) (layer "B.Cu") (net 2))
 (segment (start 67.083 63.568) (end 64.402 66.249) (width 0.25) (layer "B.Cu") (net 2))
 (segment (start 49.317 70.378) (end 52.808 73.869) (width 0.25) (layer "B.Cu") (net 16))
 (segment (start 52.808 73.869) (end 56.782 73.869) (width 0.25) (layer "B.Cu") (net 16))
 (segment (start 49.317 70.378) (end 50.492 69.203) (width 0.25) (layer "B.Cu") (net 16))
 (segment (start 50.492 67.459) (end 56.782 61.169) (width 0.25) (layer "B.Cu") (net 16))
 (segment (start 50.492 69.203) (end 50.492 67.459) (width 0.25) (layer "B.Cu") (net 16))
 (segment (start 67.083 65.772) (end 64.402 68.453) (width 0.25) (layer "B.Cu") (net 1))
 (segment (start 64.402 68.453) (end 64.402 68.789) (width 0.25) (layer "B.Cu") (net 1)))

